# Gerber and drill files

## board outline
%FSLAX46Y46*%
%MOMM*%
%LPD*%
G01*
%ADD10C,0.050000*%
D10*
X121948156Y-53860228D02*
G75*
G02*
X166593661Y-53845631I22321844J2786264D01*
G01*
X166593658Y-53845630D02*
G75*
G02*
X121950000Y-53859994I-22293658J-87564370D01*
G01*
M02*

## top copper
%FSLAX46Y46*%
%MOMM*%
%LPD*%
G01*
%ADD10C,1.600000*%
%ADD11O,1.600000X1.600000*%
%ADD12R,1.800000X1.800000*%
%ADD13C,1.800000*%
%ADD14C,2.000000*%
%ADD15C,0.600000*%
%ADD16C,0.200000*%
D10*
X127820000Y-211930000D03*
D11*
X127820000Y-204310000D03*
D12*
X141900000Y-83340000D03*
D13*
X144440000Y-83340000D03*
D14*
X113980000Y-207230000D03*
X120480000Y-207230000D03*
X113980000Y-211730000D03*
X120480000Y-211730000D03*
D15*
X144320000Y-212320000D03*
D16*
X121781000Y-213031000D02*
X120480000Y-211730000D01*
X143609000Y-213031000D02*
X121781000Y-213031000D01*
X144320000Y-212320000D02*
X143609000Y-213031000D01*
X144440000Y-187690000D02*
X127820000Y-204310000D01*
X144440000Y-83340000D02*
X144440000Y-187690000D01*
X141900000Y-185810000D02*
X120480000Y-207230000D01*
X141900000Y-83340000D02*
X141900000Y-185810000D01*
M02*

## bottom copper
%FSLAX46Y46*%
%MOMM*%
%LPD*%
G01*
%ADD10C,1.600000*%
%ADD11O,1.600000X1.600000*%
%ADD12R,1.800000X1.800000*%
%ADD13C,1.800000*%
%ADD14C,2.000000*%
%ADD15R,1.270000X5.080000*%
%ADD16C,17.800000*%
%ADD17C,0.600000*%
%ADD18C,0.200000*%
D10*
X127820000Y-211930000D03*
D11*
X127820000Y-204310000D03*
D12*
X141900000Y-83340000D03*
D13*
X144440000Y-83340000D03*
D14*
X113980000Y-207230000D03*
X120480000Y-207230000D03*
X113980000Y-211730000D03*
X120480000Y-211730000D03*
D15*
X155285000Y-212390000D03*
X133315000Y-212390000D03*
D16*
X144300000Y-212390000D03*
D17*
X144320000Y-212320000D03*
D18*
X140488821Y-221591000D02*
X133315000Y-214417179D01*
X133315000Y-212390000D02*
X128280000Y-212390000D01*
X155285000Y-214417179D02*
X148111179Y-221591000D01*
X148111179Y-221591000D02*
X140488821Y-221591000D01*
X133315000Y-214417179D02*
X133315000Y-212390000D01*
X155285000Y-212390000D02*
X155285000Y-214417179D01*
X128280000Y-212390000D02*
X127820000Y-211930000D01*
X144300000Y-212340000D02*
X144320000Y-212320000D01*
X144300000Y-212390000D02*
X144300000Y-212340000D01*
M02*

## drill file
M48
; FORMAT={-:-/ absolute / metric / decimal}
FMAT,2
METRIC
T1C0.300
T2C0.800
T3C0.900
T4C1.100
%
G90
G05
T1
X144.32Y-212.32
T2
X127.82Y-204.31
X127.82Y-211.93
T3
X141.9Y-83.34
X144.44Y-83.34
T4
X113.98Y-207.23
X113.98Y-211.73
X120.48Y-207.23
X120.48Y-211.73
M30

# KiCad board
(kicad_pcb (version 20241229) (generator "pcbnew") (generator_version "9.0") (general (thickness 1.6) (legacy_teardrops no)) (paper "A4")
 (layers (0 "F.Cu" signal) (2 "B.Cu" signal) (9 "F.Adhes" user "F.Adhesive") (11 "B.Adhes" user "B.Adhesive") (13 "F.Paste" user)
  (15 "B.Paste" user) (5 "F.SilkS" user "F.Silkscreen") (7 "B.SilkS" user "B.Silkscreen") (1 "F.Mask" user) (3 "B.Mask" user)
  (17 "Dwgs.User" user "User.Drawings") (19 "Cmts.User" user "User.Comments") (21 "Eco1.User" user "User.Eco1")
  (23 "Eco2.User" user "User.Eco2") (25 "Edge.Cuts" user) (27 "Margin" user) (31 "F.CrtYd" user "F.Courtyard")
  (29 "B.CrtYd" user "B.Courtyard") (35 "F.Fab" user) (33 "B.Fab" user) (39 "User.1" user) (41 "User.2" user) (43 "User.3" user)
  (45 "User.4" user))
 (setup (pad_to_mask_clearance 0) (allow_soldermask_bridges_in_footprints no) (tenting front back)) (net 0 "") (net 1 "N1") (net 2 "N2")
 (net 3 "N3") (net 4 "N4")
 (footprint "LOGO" (layer "F.Cu") (at 144.3 141.41)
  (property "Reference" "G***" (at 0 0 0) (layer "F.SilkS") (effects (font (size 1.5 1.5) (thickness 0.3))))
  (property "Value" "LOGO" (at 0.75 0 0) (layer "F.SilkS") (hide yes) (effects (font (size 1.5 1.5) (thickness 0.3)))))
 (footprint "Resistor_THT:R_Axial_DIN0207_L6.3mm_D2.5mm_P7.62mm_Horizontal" (layer "F.Cu") (at 127.82 211.93 90)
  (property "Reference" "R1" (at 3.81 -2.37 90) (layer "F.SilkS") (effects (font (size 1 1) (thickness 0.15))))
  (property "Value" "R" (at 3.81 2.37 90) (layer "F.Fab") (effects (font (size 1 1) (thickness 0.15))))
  (pad "1" thru_hole circle (at 0 0 90) (size 1.6 1.6) (drill 0.8) (layers "*.Cu" "*.Mask") (remove_unused_layers no) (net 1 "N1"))
  (pad "2" thru_hole oval (at 7.62 0 90) (size 1.6 1.6) (drill 0.8) (layers "*.Cu" "*.Mask") (remove_unused_layers no) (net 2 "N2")))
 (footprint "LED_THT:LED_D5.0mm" (layer "F.Cu") (at 141.9 83.34)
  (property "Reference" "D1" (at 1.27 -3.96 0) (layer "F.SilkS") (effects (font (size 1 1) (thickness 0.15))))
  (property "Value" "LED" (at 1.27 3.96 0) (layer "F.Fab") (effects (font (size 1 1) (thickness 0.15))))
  (pad "1" thru_hole rect (at 0 0) (size 1.8 1.8) (drill 0.9) (layers "*.Cu" "*.Mask") (remove_unused_layers no) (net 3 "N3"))
  (pad "2" thru_hole circle (at 2.54 0) (size 1.8 1.8) (drill 0.9) (layers "*.Cu" "*.Mask") (remove_unused_layers no) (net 2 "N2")))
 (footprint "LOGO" (layer "F.Cu") (at 146.39 95.76)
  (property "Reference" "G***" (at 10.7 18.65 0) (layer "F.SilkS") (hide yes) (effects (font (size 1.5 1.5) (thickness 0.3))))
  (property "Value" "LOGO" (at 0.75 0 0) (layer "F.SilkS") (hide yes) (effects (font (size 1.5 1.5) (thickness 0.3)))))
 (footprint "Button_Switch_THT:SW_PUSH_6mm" (layer "F.Cu") (at 113.98 207.23)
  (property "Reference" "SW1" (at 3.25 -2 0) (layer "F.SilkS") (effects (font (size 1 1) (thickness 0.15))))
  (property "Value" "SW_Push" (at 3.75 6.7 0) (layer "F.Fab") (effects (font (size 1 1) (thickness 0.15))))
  (pad "1" thru_hole circle (at 0 0 90) (size 2 2) (drill 1.1) (layers "*.Cu" "*.Mask") (remove_unused_layers no) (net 3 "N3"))
  (pad "1" thru_hole circle (at 6.5 0 90) (size 2 2) (drill 1.1) (layers "*.Cu" "*.Mask") (remove_unused_layers no) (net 3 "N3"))
  (pad "2" thru_hole circle (at 0 4.5 90) (size 2 2) (drill 1.1) (layers "*.Cu" "*.Mask") (remove_unused_layers no) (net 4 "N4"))
  (pad "2" thru_hole circle (at 6.5 4.5 90) (size 2 2) (drill 1.1) (layers "*.Cu" "*.Mask") (remove_unused_layers no) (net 4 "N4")))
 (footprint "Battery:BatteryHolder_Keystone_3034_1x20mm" (layer "B.Cu") (at 144.3 212.39 180)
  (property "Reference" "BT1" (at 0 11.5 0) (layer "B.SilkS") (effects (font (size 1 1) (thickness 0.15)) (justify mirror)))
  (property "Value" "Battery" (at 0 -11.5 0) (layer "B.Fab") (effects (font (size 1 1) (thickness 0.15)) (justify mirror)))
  (pad "1" smd rect (at -10.985 0 180) (size 1.27 5.08) (layers "B.Cu" "B.Mask" "B.Paste") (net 1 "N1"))
  (pad "1" smd rect (at 10.985 0 180) (size 1.27 5.08) (layers "B.Cu" "B.Mask" "B.Paste") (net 1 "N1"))
  (pad "2" smd circle (at 0 0 180) (size 17.8 17.8) (layers "B.Cu" "B.Mask") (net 4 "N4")))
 (gr_arc (start 121.948156 53.860228) (mid 144.262645 28.5789) (end 166.593661 53.845631) (stroke (width 0.05) (type default))
  (layer "Edge.Cuts"))
 (gr_arc (start 166.593658 53.84563) (mid 144.329072 231.767762) (end 121.95 53.859994) (stroke (width 0.05) (type default))
  (layer "Edge.Cuts"))
 (segment (start 140.488821 221.591) (end 133.315 214.417179) (width 0.2) (layer "B.Cu") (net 1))
 (segment (start 133.315 212.39) (end 128.28 212.39) (width 0.2) (layer "B.Cu") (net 1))
 (segment (start 155.285 214.417179) (end 148.111179 221.591) (width 0.2) (layer "B.Cu") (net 1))
 (segment (start 148.111179 221.591) (end 140.488821 221.591) (width 0.2) (layer "B.Cu") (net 1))
 (segment (start 133.315 214.417179) (end 133.315 212.39) (width 0.2) (layer "B.Cu") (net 1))
 (segment (start 155.285 212.39) (end 155.285 214.417179) (width 0.2) (layer "B.Cu") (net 1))
 (segment (start 128.28 212.39) (end 127.82 211.93) (width 0.2) (layer "B.Cu") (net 1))
 (segment (start 121.781 213.031) (end 120.48 211.73) (width 0.2) (layer "F.Cu") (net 4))
 (segment (start 143.609 213.031) (end 121.781 213.031) (width 0.2) (layer "F.Cu") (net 4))
 (segment (start 144.32 212.32) (end 143.609 213.031) (width 0.2) (layer "F.Cu") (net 4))
 (via (at 144.32 212.32) (size 0.6) (drill 0.3) (layers "F.Cu" "B.Cu") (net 4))
 (segment (start 144.3 212.34) (end 144.32 212.32) (width 0.2) (layer "B.Cu") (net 4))
 (segment (start 144.3 212.39) (end 144.3 212.34) (width 0.2) (layer "B.Cu") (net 4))
 (segment (start 144.44 187.69) (end 127.82 204.31) (width 0.2) (layer "F.Cu") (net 2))
 (segment (start 144.44 83.34) (end 144.44 187.69) (width 0.2) (layer "F.Cu") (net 2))
 (segment (start 141.9 185.81) (end 120.48 207.23) (width 0.2) (layer "F.Cu") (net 3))
 (segment (start 141.9 83.34) (end 141.9 185.81) (width 0.2) (layer "F.Cu") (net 3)))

